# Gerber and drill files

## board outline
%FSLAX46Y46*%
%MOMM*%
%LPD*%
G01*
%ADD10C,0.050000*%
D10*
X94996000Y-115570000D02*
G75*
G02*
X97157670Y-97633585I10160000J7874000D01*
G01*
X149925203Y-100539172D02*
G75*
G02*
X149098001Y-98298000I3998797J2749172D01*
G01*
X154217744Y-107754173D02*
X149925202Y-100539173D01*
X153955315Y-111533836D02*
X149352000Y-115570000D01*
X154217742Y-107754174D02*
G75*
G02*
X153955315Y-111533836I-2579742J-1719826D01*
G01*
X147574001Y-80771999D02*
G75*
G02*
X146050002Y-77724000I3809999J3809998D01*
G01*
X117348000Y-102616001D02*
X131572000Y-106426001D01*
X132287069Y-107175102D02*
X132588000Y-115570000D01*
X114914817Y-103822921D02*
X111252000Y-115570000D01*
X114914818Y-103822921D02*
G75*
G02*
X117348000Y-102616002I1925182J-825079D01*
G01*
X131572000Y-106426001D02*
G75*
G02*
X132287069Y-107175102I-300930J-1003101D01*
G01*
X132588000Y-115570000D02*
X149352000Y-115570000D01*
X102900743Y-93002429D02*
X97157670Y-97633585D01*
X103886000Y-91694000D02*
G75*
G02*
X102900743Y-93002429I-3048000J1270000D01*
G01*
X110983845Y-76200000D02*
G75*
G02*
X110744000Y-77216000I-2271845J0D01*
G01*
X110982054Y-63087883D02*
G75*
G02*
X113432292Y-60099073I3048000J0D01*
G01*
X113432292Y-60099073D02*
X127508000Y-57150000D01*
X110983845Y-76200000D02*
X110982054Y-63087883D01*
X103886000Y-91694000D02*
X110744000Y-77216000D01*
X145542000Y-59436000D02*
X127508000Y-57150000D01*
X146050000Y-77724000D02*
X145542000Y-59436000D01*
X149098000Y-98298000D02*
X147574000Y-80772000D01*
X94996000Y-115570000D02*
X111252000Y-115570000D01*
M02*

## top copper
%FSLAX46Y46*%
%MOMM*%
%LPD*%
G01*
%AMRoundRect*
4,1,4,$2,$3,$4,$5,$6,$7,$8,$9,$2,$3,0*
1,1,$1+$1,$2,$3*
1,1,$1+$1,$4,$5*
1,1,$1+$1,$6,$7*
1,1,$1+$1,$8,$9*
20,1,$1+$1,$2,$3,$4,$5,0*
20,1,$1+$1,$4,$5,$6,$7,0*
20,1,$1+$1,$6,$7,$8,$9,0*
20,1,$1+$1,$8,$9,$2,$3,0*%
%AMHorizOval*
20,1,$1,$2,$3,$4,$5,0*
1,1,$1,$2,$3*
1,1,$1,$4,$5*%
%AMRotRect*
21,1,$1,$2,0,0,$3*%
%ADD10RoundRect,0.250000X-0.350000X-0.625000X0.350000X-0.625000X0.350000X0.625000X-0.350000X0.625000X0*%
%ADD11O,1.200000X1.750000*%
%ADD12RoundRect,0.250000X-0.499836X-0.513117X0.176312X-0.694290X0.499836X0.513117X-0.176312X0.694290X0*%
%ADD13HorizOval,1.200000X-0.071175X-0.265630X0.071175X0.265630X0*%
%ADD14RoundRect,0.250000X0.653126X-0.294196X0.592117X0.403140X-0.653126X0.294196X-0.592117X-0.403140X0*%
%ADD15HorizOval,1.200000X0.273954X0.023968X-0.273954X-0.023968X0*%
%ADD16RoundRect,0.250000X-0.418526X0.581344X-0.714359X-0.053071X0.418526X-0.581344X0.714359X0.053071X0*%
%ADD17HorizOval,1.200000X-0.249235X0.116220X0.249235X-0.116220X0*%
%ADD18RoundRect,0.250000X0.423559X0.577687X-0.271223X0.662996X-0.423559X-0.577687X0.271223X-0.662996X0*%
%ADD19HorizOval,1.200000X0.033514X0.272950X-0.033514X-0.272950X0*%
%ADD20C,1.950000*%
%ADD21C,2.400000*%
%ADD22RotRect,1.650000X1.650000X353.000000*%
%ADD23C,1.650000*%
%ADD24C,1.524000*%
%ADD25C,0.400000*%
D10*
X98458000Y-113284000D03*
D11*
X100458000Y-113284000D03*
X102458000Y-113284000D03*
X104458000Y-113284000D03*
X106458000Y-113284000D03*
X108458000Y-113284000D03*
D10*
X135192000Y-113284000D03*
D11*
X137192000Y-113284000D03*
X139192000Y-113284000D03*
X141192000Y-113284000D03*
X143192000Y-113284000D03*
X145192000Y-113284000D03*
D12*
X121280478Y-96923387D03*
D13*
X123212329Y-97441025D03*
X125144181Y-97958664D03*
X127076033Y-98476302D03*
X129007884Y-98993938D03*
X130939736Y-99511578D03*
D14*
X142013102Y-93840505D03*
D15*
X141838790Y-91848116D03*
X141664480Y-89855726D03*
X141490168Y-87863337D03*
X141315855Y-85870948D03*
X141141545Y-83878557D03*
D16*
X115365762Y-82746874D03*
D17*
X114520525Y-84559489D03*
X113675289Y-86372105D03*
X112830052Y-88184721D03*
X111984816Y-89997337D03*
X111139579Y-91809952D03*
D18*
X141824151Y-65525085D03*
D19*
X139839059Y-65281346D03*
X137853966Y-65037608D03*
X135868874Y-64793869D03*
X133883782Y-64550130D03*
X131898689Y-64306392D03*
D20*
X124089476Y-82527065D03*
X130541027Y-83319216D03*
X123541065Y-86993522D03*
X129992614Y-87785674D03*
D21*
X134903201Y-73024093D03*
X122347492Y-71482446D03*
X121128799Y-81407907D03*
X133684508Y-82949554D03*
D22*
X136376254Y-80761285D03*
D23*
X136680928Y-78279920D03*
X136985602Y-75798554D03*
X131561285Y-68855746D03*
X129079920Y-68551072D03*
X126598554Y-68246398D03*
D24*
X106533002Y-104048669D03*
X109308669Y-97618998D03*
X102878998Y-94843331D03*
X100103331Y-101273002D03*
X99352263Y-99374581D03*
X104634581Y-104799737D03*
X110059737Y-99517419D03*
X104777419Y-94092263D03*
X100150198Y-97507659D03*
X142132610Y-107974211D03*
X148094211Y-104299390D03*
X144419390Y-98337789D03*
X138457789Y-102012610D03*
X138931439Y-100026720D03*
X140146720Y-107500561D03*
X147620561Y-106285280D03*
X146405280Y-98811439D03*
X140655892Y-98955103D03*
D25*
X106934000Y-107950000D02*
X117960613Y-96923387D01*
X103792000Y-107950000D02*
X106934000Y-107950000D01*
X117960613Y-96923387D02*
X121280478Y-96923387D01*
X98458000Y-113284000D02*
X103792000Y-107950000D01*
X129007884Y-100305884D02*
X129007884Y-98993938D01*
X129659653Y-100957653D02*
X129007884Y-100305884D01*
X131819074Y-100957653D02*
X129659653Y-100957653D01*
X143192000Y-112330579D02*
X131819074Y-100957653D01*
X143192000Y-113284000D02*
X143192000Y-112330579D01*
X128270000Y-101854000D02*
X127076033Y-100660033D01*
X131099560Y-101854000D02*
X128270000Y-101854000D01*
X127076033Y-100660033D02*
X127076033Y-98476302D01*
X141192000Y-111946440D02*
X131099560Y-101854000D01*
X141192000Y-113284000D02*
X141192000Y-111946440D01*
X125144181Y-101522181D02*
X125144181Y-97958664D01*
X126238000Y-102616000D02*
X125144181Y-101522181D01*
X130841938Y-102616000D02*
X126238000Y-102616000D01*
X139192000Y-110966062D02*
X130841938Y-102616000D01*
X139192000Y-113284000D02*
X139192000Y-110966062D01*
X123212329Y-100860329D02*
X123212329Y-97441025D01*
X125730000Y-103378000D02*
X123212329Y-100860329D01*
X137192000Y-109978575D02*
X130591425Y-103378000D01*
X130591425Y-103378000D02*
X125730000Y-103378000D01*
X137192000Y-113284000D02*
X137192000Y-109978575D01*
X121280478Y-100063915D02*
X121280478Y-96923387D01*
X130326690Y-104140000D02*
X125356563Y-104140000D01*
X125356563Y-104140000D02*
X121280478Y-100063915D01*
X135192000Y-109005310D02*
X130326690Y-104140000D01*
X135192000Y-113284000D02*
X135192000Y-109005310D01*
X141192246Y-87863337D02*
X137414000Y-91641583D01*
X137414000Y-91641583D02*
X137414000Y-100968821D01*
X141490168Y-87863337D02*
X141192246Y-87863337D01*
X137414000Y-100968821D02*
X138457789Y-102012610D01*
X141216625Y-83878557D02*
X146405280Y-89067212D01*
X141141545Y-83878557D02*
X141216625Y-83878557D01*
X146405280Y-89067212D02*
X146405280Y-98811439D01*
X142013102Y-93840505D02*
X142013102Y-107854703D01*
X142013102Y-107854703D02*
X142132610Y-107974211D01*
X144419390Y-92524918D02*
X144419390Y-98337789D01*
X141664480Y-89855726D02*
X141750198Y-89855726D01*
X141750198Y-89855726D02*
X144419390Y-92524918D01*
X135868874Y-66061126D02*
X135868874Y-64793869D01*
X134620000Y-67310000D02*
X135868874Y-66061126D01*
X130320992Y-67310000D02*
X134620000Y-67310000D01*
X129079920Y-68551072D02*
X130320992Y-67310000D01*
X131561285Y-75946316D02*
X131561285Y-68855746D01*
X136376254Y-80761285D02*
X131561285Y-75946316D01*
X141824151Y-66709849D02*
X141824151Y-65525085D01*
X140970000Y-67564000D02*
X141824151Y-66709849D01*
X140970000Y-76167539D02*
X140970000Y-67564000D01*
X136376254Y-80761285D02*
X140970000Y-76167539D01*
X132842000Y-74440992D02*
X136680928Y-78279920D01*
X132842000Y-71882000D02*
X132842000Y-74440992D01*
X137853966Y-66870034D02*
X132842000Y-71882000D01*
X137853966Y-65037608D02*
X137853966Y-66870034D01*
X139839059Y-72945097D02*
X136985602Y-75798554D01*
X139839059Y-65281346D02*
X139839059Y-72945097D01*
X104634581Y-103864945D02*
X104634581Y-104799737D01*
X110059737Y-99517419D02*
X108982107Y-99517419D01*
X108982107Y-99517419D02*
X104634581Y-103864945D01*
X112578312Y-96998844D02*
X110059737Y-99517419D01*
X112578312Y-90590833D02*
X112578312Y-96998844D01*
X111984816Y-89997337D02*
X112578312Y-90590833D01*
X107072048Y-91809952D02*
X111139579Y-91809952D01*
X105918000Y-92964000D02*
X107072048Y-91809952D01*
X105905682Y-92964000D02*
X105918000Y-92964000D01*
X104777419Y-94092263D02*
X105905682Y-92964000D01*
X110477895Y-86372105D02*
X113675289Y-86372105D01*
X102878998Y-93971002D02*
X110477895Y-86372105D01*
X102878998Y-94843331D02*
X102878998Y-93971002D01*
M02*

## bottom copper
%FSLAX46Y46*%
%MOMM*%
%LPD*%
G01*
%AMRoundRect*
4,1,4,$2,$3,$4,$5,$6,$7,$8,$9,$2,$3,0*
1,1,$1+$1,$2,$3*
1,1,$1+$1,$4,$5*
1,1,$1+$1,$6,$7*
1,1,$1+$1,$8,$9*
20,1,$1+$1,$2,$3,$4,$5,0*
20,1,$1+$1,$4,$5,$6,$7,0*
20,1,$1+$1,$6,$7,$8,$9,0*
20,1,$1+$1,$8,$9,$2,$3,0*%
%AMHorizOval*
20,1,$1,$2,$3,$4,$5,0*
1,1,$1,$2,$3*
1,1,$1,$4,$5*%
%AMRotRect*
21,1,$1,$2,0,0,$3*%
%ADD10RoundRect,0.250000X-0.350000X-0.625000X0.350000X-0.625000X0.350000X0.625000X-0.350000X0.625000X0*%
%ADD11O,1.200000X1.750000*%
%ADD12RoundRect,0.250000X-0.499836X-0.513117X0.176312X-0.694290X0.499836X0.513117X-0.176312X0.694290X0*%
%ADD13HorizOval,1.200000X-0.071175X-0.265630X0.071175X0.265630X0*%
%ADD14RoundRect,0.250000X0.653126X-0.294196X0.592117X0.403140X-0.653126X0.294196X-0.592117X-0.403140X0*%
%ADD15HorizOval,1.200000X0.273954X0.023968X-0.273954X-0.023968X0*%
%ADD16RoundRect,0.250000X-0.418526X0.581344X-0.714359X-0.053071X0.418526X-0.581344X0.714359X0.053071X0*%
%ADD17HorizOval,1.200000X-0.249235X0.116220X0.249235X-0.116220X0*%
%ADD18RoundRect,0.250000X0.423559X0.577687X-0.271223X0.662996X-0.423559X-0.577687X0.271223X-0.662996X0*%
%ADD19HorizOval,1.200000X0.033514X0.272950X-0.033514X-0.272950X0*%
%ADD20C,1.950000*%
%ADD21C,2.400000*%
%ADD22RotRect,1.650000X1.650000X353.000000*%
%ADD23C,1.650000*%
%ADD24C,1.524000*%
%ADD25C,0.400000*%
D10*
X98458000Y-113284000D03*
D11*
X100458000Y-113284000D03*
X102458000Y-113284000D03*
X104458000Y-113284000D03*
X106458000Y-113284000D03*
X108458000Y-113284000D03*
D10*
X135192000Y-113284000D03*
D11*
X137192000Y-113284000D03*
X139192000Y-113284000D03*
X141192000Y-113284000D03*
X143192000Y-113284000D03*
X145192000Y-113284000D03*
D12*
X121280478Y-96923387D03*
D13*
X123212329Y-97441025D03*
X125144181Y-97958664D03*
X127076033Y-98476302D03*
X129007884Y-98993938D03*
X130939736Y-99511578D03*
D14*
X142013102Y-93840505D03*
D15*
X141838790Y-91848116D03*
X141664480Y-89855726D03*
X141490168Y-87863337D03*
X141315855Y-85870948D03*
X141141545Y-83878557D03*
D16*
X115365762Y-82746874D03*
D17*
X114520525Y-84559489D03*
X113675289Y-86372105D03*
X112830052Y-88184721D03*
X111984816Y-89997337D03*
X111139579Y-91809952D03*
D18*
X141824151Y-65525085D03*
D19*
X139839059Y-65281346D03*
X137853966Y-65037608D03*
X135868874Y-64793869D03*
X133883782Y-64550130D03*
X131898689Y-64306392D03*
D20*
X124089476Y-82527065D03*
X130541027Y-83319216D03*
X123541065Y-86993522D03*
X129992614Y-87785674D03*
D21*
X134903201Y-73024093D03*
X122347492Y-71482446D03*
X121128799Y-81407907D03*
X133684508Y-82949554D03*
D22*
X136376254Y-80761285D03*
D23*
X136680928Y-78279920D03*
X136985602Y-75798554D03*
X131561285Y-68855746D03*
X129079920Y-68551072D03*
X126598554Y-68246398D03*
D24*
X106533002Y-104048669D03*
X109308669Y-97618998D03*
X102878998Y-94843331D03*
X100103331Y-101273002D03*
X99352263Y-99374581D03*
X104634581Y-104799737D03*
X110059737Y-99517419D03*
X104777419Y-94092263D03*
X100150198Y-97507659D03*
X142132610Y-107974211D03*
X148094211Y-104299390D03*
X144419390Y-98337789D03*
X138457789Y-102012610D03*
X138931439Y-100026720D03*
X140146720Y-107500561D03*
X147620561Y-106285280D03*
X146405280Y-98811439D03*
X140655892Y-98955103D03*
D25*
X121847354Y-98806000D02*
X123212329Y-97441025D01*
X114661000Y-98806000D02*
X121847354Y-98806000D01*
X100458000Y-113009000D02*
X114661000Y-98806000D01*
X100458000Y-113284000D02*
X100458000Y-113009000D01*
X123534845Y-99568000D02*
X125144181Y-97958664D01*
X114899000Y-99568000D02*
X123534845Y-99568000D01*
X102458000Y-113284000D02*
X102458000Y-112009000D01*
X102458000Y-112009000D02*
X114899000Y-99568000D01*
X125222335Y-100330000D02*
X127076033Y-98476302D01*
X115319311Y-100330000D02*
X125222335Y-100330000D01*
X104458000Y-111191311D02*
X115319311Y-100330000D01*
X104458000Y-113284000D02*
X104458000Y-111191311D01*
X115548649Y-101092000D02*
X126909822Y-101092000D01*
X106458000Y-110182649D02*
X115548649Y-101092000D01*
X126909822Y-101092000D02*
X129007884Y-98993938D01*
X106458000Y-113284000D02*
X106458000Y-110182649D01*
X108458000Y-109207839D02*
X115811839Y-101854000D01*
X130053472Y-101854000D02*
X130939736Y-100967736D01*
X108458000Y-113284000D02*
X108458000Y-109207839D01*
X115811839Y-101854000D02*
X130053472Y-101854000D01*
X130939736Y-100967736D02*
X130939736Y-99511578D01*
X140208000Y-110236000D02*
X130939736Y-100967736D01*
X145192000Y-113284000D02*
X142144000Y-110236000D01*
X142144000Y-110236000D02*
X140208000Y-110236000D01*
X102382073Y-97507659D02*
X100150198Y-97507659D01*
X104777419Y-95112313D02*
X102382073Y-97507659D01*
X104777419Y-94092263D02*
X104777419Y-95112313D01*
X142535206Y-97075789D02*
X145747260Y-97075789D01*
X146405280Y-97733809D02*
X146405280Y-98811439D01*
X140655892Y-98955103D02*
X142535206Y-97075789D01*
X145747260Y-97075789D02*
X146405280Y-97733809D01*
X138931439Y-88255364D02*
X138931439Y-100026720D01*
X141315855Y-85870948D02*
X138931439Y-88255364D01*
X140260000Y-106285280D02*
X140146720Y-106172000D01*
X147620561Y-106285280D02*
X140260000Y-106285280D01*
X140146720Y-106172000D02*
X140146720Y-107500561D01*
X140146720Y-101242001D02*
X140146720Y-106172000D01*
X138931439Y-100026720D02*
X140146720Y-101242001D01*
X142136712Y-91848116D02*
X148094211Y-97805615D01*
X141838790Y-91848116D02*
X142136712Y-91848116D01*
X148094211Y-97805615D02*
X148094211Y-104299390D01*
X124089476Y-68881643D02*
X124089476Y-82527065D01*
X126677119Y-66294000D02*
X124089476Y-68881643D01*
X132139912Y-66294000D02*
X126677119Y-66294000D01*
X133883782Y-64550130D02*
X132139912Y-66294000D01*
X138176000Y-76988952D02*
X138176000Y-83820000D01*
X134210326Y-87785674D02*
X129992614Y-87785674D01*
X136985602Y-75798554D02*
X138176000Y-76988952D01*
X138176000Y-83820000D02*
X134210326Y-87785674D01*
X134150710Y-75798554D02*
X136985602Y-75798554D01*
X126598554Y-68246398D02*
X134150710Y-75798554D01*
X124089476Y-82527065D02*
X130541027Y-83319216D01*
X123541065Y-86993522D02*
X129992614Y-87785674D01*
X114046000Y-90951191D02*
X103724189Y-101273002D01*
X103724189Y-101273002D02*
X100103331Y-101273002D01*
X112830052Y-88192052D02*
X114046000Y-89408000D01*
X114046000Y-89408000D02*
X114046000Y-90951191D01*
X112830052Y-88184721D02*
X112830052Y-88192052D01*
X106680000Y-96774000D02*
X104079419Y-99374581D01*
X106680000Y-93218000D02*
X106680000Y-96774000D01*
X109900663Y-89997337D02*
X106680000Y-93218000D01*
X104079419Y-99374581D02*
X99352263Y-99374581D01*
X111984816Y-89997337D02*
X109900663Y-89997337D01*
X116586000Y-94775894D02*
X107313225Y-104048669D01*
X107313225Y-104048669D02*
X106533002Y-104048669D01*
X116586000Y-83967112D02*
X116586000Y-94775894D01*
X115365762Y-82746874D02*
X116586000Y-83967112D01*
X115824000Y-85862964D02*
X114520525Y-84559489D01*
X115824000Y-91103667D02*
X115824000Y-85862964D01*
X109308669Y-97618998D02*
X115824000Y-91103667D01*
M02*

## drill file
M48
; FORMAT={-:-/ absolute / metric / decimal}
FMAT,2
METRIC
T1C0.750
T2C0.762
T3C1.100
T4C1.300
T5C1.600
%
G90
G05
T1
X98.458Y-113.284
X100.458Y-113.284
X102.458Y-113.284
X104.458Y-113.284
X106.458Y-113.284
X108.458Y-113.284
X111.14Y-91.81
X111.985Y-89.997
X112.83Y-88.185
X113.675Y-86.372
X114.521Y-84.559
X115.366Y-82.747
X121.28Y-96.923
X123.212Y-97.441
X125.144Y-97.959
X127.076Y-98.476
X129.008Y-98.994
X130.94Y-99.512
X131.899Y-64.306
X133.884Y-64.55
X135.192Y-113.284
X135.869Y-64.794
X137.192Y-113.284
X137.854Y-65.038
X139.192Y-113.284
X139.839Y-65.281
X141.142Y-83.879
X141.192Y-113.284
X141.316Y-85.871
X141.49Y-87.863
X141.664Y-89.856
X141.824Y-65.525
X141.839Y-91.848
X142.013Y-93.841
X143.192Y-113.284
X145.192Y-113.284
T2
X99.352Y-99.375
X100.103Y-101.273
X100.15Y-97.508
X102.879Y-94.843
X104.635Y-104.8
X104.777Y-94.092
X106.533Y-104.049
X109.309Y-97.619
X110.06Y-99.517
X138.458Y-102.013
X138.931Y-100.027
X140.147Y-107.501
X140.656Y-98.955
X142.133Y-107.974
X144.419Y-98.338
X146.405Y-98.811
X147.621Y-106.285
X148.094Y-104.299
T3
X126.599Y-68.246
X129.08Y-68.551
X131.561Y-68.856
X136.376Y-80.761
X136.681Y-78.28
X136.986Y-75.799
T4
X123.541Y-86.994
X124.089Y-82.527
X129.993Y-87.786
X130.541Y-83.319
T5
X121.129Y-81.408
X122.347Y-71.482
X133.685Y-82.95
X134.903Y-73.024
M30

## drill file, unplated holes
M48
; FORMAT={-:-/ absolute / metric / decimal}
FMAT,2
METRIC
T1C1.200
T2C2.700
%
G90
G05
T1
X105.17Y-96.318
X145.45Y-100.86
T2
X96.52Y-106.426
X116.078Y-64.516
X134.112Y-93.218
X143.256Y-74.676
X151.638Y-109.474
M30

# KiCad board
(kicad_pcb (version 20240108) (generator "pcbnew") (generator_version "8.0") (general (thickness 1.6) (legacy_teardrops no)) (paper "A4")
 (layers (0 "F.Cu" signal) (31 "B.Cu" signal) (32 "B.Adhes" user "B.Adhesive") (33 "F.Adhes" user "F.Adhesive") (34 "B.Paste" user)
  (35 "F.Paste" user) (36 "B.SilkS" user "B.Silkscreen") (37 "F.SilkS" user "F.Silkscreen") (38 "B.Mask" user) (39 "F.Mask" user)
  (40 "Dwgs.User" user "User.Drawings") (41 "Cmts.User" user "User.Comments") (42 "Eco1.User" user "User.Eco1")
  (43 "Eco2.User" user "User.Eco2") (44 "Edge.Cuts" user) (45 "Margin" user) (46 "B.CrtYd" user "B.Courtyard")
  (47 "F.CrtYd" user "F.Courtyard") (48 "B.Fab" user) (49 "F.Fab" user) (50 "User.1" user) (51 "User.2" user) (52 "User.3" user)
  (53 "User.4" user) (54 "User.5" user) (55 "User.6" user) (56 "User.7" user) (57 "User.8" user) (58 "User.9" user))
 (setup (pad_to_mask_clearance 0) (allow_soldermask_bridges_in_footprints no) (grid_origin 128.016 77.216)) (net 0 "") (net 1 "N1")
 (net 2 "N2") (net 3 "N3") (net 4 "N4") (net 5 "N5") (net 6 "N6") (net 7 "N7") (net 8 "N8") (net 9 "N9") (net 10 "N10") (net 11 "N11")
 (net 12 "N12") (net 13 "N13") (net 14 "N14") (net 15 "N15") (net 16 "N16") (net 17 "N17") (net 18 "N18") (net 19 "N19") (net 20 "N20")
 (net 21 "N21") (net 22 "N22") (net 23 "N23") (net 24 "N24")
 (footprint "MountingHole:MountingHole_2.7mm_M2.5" (layer "F.Cu") (at 151.638 109.474)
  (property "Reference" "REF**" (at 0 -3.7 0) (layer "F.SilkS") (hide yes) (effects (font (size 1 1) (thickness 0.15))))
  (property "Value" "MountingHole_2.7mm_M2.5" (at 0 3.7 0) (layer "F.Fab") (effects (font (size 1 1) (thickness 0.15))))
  (pad "" np_thru_hole circle (at 0 0) (size 2.7 2.7) (drill 2.7) (layers "*.Cu" "*.Mask")))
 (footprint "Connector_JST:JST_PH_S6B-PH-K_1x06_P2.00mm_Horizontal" (layer "F.Cu") (at 121.280478 96.923387 -15)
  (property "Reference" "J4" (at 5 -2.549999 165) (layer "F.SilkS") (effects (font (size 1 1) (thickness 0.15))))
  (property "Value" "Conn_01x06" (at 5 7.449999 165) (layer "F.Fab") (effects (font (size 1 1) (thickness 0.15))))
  (pad "1" thru_hole roundrect (at 0 0 345) (size 1.2 1.75) (drill 0.75) (layers "*.Cu" "*.Mask") (remove_unused_layers no)
   (roundrect_rratio 0.208333) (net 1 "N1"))
  (pad "2" thru_hole oval (at 1.999999 0 345) (size 1.2 1.75) (drill 0.75) (layers "*.Cu" "*.Mask") (remove_unused_layers no) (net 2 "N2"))
  (pad "3" thru_hole oval (at 4 0.000001 345) (size 1.2 1.75) (drill 0.75) (layers "*.Cu" "*.Mask") (remove_unused_layers no) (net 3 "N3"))
  (pad "4" thru_hole oval (at 6 0.000001 345) (size 1.2 1.75) (drill 0.75) (layers "*.Cu" "*.Mask") (remove_unused_layers no) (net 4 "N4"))
  (pad "5" thru_hole oval (at 7.999999 -0.000001 345) (size 1.2 1.75) (drill 0.75) (layers "*.Cu" "*.Mask") (remove_unused_layers no)
   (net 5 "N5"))
  (pad "6" thru_hole oval (at 10 0.000001 345) (size 1.2 1.75) (drill 0.75) (layers "*.Cu" "*.Mask") (remove_unused_layers no) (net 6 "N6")))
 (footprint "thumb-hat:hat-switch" (layer "F.Cu") (at 104.706 99.446 10)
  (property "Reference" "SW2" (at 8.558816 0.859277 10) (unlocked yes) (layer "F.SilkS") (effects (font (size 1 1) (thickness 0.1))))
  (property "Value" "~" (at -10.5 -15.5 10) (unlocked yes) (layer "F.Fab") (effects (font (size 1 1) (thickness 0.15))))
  (pad "" np_thru_hole circle (at 1.000001 -2.999999 10) (size 1.2 1.2) (drill 1.2) (layers "*.Mask"))
  (pad "1" thru_hole circle (at 1.000001 4.85 10) (size 1.524 1.524) (drill 0.762) (layers "*.Cu" "*.Mask") (remove_unused_layers no)
   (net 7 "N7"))
  (pad "2" thru_hole circle (at 4.85 -1.000001 10) (size 1.524 1.524) (drill 0.762) (layers "*.Cu" "*.Mask") (remove_unused_layers no)
   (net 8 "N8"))
  (pad "3" thru_hole circle (at -1.000001 -4.85 10) (size 1.524 1.524) (drill 0.762) (layers "*.Cu" "*.Mask") (remove_unused_layers no)
   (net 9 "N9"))
  (pad "4" thru_hole circle (at -4.85 1.000001 10) (size 1.524 1.524) (drill 0.762) (layers "*.Cu" "*.Mask") (remove_unused_layers no)
   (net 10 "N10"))
  (pad "5" thru_hole circle (at -5.26 -1.000001 10) (size 1.524 1.524) (drill 0.762) (layers "*.Cu" "*.Mask") (remove_unused_layers no)
   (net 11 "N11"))
  (pad "5" thru_hole circle (at -1.000001 5.26 10) (size 1.524 1.524) (drill 0.762) (layers "*.Cu" "*.Mask") (remove_unused_layers no)
   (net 11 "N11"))
  (pad "5" thru_hole circle (at 5.26 1.000001 10) (size 1.524 1.524) (drill 0.762) (layers "*.Cu" "*.Mask") (remove_unused_layers no)
   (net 11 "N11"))
  (pad "6" thru_hole circle (at 1.000001 -5.26 10) (size 1.524 1.524) (drill 0.762) (layers "*.Cu" "*.Mask") (remove_unused_layers no)
   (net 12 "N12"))
  (pad "7" thru_hole circle (at -4.15 -2.7 10) (size 1.524 1.524) (drill 0.762) (layers "*.Cu" "*.Mask") (remove_unused_layers no)
   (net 12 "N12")))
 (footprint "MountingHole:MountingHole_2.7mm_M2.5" (layer "F.Cu") (at 116.078 64.516)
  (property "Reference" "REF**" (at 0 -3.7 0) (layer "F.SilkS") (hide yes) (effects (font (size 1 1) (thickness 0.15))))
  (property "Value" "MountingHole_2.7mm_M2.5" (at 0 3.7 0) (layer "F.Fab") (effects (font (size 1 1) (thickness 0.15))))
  (pad "" np_thru_hole circle (at 0 0) (size 2.7 2.7) (drill 2.7) (layers "*.Cu" "*.Mask")))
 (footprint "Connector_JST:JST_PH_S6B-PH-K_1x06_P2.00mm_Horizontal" (layer "F.Cu") (at 141.824151 65.525085 173)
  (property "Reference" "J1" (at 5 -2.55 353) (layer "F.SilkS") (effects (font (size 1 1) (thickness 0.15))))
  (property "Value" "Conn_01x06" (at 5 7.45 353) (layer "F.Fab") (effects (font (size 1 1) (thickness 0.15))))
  (pad "1" thru_hole roundrect (at 0 0 173) (size 1.2 1.75) (drill 0.75) (layers "*.Cu" "*.Mask") (remove_unused_layers no)
   (roundrect_rratio 0.208333) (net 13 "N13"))
  (pad "2" thru_hole oval (at 2 0 173) (size 1.2 1.75) (drill 0.75) (layers "*.Cu" "*.Mask") (remove_unused_layers no) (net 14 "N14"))
  (pad "3" thru_hole oval (at 4 0 173) (size 1.2 1.75) (drill 0.75) (layers "*.Cu" "*.Mask") (remove_unused_layers no) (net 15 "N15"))
  (pad "4" thru_hole oval (at 6 0 173) (size 1.2 1.75) (drill 0.75) (layers "*.Cu" "*.Mask") (remove_unused_layers no) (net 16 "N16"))
  (pad "5" thru_hole oval (at 8 0 173) (size 1.2 1.75) (drill 0.75) (layers "*.Cu" "*.Mask") (remove_unused_layers no) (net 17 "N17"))
  (pad "6" thru_hole oval (at 10 0 173) (size 1.2 1.75) (drill 0.75) (layers "*.Cu" "*.Mask") (remove_unused_layers no) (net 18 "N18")))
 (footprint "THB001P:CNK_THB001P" (layer "F.Cu") (at 128.016 77.216 -7)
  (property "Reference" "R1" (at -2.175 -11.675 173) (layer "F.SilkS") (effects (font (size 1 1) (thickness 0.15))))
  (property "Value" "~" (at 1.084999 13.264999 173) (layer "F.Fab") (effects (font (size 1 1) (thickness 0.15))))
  (pad "A" thru_hole circle (at -3.25 5.75 353) (size 1.95 1.95) (drill 1.3) (layers "*.Cu" "*.Mask") (remove_unused_layers no)
   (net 17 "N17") (solder_mask_margin 0.102))
  (pad "B" thru_hole circle (at 3.250001 5.75 353) (size 1.95 1.95) (drill 1.3) (layers "*.Cu" "*.Mask") (remove_unused_layers no)
   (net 17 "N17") (solder_mask_margin 0.102))
  (pad "C" thru_hole circle (at -3.249999 10.249999 353) (size 1.95 1.95) (drill 1.3) (layers "*.Cu" "*.Mask") (remove_unused_layers no)
   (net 14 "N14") (solder_mask_margin 0.102))
  (pad "D" thru_hole circle (at 3.25 10.250001 353) (size 1.95 1.95) (drill 1.3) (layers "*.Cu" "*.Mask") (remove_unused_layers no)
   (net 14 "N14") (solder_mask_margin 0.102))
  (pad "S1" thru_hole circle (at 6.325 -5 353) (size 2.4 2.4) (drill 1.6) (layers "*.Cu" "*.Mask") (remove_unused_layers no)
   (solder_mask_margin 0.102))
  (pad "S2" thru_hole circle (at -6.325 -5 353) (size 2.4 2.4) (drill 1.6) (layers "*.Cu" "*.Mask") (remove_unused_layers no)
   (solder_mask_margin 0.102))
  (pad "S3" thru_hole circle (at -6.325 5 353) (size 2.4 2.4) (drill 1.6) (layers "*.Cu" "*.Mask") (remove_unused_layers no)
   (solder_mask_margin 0.102))
  (pad "S4" thru_hole circle (at 6.325 5 353) (size 2.4 2.4) (drill 1.6) (layers "*.Cu" "*.Mask") (remove_unused_layers no)
   (solder_mask_margin 0.102))
  (pad "VR1_1" thru_hole rect (at 8.729999 2.5 353) (size 1.65 1.65) (drill 1.1) (layers "*.Cu" "*.Mask") (remove_unused_layers no)
   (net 13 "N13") (solder_mask_margin 0.102))
  (pad "VR1_2" thru_hole circle (at 8.73 0.000001 353) (size 1.65 1.65) (drill 1.1) (layers "*.Cu" "*.Mask") (remove_unused_layers no)
   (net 15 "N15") (solder_mask_margin 0.102))
  (pad "VR1_3" thru_hole circle (at 8.730001 -2.5 353) (size 1.65 1.65) (drill 1.1) (layers "*.Cu" "*.Mask") (remove_unused_layers no)
   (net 14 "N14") (solder_mask_margin 0.102))
  (pad "VR2_1" thru_hole circle (at 2.5 -8.729999 353) (size 1.65 1.65) (drill 1.1) (layers "*.Cu" "*.Mask") (remove_unused_layers no)
   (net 13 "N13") (solder_mask_margin 0.102))
  (pad "VR2_2" thru_hole circle (at 0.000001 -8.73 353) (size 1.65 1.65) (drill 1.1) (layers "*.Cu" "*.Mask") (remove_unused_layers no)
   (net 16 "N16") (solder_mask_margin 0.102))
  (pad "VR2_3" thru_hole circle (at -2.5 -8.730001 353) (size 1.65 1.65) (drill 1.1) (layers "*.Cu" "*.Mask") (remove_unused_layers no)
   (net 14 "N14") (solder_mask_margin 0.102)))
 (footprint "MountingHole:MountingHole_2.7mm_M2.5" (layer "F.Cu") (at 134.112 93.218)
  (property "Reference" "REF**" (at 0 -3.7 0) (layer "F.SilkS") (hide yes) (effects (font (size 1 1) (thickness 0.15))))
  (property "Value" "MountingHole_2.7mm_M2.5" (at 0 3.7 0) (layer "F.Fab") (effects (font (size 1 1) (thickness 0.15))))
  (pad "" np_thru_hole circle (at 0 0) (size 2.7 2.7) (drill 2.7) (layers "*.Cu" "*.Mask")))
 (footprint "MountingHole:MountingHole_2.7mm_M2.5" (layer "F.Cu") (at 96.52 106.426)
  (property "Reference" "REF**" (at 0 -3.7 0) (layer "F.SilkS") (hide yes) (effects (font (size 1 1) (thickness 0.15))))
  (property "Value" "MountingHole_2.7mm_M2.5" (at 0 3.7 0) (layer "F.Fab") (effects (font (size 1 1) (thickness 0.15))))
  (pad "" np_thru_hole circle (at 0 0) (size 2.7 2.7) (drill 2.7) (layers "*.Cu" "*.Mask")))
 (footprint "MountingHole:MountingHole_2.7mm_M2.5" (layer "F.Cu") (at 143.256 74.676)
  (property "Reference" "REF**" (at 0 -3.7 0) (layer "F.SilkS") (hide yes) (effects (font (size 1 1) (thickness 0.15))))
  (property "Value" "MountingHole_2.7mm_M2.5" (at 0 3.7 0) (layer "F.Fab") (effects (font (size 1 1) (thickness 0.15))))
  (pad "" np_thru_hole circle (at 0 0) (size 2.7 2.7) (drill 2.7) (layers "*.Cu" "*.Mask")))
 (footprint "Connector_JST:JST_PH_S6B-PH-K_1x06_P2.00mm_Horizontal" (layer "F.Cu") (at 115.365762 82.746874 -115)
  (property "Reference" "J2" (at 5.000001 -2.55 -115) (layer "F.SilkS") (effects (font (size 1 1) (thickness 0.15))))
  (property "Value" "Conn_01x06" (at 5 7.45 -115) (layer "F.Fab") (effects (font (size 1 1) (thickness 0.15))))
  (pad "1" thru_hole roundrect (at 0 0 245) (size 1.2 1.75) (drill 0.75) (layers "*.Cu" "*.Mask") (remove_unused_layers no)
   (roundrect_rratio 0.208333) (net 7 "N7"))
  (pad "2" thru_hole oval (at 2 0.000001 245) (size 1.2 1.75) (drill 0.75) (layers "*.Cu" "*.Mask") (remove_unused_layers no) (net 8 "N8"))
  (pad "3" thru_hole oval (at 4 0 245) (size 1.2 1.75) (drill 0.75) (layers "*.Cu" "*.Mask") (remove_unused_layers no) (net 9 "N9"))
  (pad "4" thru_hole oval (at 6 0 245) (size 1.2 1.75) (drill 0.75) (layers "*.Cu" "*.Mask") (remove_unused_layers no) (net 10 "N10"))
  (pad "5" thru_hole oval (at 8.000001 0 245) (size 1.2 1.75) (drill 0.75) (layers "*.Cu" "*.Mask") (remove_unused_layers no) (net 11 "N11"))
  (pad "6" thru_hole oval (at 10 0 245) (size 1.2 1.75) (drill 0.75) (layers "*.Cu" "*.Mask") (remove_unused_layers no) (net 12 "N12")))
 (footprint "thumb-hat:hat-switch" (layer "F.Cu") (at 143.276 103.156 -25)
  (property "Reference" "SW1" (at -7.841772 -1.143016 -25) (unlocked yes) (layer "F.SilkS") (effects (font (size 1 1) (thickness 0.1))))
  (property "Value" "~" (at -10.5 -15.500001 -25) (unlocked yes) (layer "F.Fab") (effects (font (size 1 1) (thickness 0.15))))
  (pad "" np_thru_hole circle (at 1 -3 335) (size 1.2 1.2) (drill 1.2) (layers "*.Mask"))
  (pad "1" thru_hole circle (at 1.000001 4.85 335) (size 1.524 1.524) (drill 0.762) (layers "*.Cu" "*.Mask") (remove_unused_layers no)
   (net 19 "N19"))
  (pad "2" thru_hole circle (at 4.85 -1.000001 335) (size 1.524 1.524) (drill 0.762) (layers "*.Cu" "*.Mask") (remove_unused_layers no)
   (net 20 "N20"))
  (pad "3" thru_hole circle (at -1.000001 -4.85 335) (size 1.524 1.524) (drill 0.762) (layers "*.Cu" "*.Mask") (remove_unused_layers no)
   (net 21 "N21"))
  (pad "4" thru_hole circle (at -4.85 1.000001 335) (size 1.524 1.524) (drill 0.762) (layers "*.Cu" "*.Mask") (remove_unused_layers no)
   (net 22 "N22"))
  (pad "5" thru_hole circle (at -5.26 -1 335) (size 1.524 1.524) (drill 0.762) (layers "*.Cu" "*.Mask") (remove_unused_layers no)
   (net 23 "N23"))
  (pad "5" thru_hole circle (at -1 5.26 335) (size 1.524 1.524) (drill 0.762) (layers "*.Cu" "*.Mask") (remove_unused_layers no)
   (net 23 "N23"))
  (pad "5" thru_hole circle (at 5.26 1 335) (size 1.524 1.524) (drill 0.762) (layers "*.Cu" "*.Mask") (remove_unused_layers no)
   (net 23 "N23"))
  (pad "6" thru_hole circle (at 1 -5.26 335) (size 1.524 1.524) (drill 0.762) (layers "*.Cu" "*.Mask") (remove_unused_layers no)
   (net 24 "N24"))
  (pad "7" thru_hole circle (at -4.15 -2.7 335) (size 1.524 1.524) (drill 0.762) (layers "*.Cu" "*.Mask") (remove_unused_layers no)
   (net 24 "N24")))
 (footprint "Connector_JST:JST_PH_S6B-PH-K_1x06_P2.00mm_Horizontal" (layer "F.Cu") (at 142.013102 93.840505 95)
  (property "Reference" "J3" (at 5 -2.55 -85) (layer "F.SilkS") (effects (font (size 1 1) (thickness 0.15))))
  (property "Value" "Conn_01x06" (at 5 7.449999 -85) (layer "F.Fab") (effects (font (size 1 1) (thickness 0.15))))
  (pad "1" thru_hole roundrect (at 0 0 95) (size 1.2 1.75) (drill 0.75) (layers "*.Cu" "*.Mask") (remove_unused_layers no)
   (roundrect_rratio 0.208333) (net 19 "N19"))
  (pad "2" thru_hole oval (at 2 -0.000001 95) (size 1.2 1.75) (drill 0.75) (layers "*.Cu" "*.Mask") (remove_unused_layers no) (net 20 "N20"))
  (pad "3" thru_hole oval (at 4 0.000001 95) (size 1.2 1.75) (drill 0.75) (layers "*.Cu" "*.Mask") (remove_unused_layers no) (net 21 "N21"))
  (pad "4" thru_hole oval (at 6 0 95) (size 1.2 1.75) (drill 0.75) (layers "*.Cu" "*.Mask") (remove_unused_layers no) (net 22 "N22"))
  (pad "5" thru_hole oval (at 8 -0.000001 95) (size 1.2 1.75) (drill 0.75) (layers "*.Cu" "*.Mask") (remove_unused_layers no) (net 23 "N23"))
  (pad "6" thru_hole oval (at 10.000001 0.000001 95) (size 1.2 1.75) (drill 0.75) (layers "*.Cu" "*.Mask") (remove_unused_layers no)
   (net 24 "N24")))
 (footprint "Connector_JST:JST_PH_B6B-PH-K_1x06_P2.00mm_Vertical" (layer "B.Cu") (at 98.458 113.284)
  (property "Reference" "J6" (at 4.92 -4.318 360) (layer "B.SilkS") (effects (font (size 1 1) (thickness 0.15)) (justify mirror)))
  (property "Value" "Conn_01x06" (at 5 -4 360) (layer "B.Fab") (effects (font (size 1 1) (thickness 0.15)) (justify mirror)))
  (pad "1" thru_hole roundrect (at 0 0) (size 1.2 1.75) (drill 0.75) (layers "*.Cu" "*.Mask") (remove_unused_layers no)
   (roundrect_rratio 0.208333) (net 1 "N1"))
  (pad "2" thru_hole oval (at 2 0) (size 1.2 1.75) (drill 0.75) (layers "*.Cu" "*.Mask") (remove_unused_layers no) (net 2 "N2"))
  (pad "3" thru_hole oval (at 4 0) (size 1.2 1.75) (drill 0.75) (layers "*.Cu" "*.Mask") (remove_unused_layers no) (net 3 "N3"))
  (pad "4" thru_hole oval (at 6 0) (size 1.2 1.75) (drill 0.75) (layers "*.Cu" "*.Mask") (remove_unused_layers no) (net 4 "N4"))
  (pad "5" thru_hole oval (at 8 0) (size 1.2 1.75) (drill 0.75) (layers "*.Cu" "*.Mask") (remove_unused_layers no) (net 5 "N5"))
  (pad "6" thru_hole oval (at 10 0) (size 1.2 1.75) (drill 0.75) (layers "*.Cu" "*.Mask") (remove_unused_layers no) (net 6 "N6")))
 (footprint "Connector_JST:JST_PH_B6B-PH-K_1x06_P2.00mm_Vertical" (layer "B.Cu") (at 135.192 113.284)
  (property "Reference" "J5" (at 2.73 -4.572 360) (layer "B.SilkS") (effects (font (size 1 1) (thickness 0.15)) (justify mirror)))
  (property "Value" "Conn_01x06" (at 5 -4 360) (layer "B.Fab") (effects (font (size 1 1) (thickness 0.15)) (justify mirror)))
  (pad "1" thru_hole roundrect (at 0 0) (size 1.2 1.75) (drill 0.75) (layers "*.Cu" "*.Mask") (remove_unused_layers no)
   (roundrect_rratio 0.208333) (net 1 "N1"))
  (pad "2" thru_hole oval (at 2 0) (size 1.2 1.75) (drill 0.75) (layers "*.Cu" "*.Mask") (remove_unused_layers no) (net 2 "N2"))
  (pad "3" thru_hole oval (at 4 0) (size 1.2 1.75) (drill 0.75) (layers "*.Cu" "*.Mask") (remove_unused_layers no) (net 3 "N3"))
  (pad "4" thru_hole oval (at 6 0) (size 1.2 1.75) (drill 0.75) (layers "*.Cu" "*.Mask") (remove_unused_layers no) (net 4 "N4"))
  (pad "5" thru_hole oval (at 8 0) (size 1.2 1.75) (drill 0.75) (layers "*.Cu" "*.Mask") (remove_unused_layers no) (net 5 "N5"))
  (pad "6" thru_hole oval (at 10 0) (size 1.2 1.75) (drill 0.75) (layers "*.Cu" "*.Mask") (remove_unused_layers no) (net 6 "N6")))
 (gr_arc (start 110.983845 76.2) (mid 110.923071 76.721963) (end 110.744 77.216) (stroke (width 0.05) (type default)) (layer "Edge.Cuts"))
 (gr_line (start 117.348 102.616001) (end 131.572 106.426001) (stroke (width 0.05) (type default)) (layer "Edge.Cuts"))
 (gr_arc (start 114.914817 103.822921) (mid 115.909266 102.771615) (end 117.348 102.616001) (stroke (width 0.05) (type default))
  (layer "Edge.Cuts"))
 (gr_line (start 146.05 77.724) (end 145.542 59.436) (stroke (width 0.05) (type default)) (layer "Edge.Cuts"))
 (gr_line (start 154.217744 107.754173) (end 149.925202 100.539173) (stroke (width 0.05) (type default)) (layer "Edge.Cuts"))
 (gr_arc (start 94.996 115.57) (mid 92.394339 106.157984) (end 97.15767 97.633585) (stroke (width 0.05) (type default)) (layer "Edge.Cuts"))
 (gr_line (start 102.900743 93.002429) (end 97.15767 97.633585) (stroke (width 0.05) (type default)) (layer "Edge.Cuts"))
 (gr_line (start 145.542 59.436) (end 127.508 57.15) (stroke (width 0.05) (type default)) (layer "Edge.Cuts"))
 (gr_arc (start 110.982054 63.087883) (mid 111.672907 61.155485) (end 113.432292 60.099073) (stroke (width 0.05) (type default))
  (layer "Edge.Cuts"))
 (gr_line (start 153.955315 111.533836) (end 149.352 115.57) (stroke (width 0.05) (type default)) (layer "Edge.Cuts"))
 (gr_arc (start 147.574 80.772) (mid 146.564689 79.371656) (end 146.050001 77.724) (stroke (width 0.05) (type default)) (layer "Edge.Cuts"))
 (gr_line (start 149.098 98.298) (end 147.574 80.772) (stroke (width 0.05) (type default)) (layer "Edge.Cuts"))
 (gr_line (start 132.588 115.57) (end 149.352 115.57) (stroke (width 0.05) (type default)) (layer "Edge.Cuts"))
 (gr_line (start 114.914817 103.822921) (end 111.252 115.57) (stroke (width 0.05) (type default)) (layer "Edge.Cuts"))
 (gr_line (start 94.996 115.57) (end 111.252 115.57) (stroke (width 0.05) (type default)) (layer "Edge.Cuts"))
 (gr_line (start 113.432292 60.099073) (end 127.508 57.15) (stroke (width 0.05) (type default)) (layer "Edge.Cuts"))
 (gr_arc (start 103.886 91.694) (mid 103.475787 92.410274) (end 102.900743 93.002429) (stroke (width 0.05) (type default))
  (layer "Edge.Cuts"))
 (gr_line (start 132.287069 107.175102) (end 132.588 115.57) (stroke (width 0.05) (type default)) (layer "Edge.Cuts"))
 (gr_line (start 103.886 91.694) (end 110.744 77.216) (stroke (width 0.05) (type default)) (layer "Edge.Cuts"))
 (gr_arc (start 154.217743 107.754174) (mid 154.731017 109.688753) (end 153.955315 111.533836) (stroke (width 0.05) (type default))
  (layer "Edge.Cuts"))
 (gr_arc (start 131.572 106.426001) (mid 132.028608 106.705979) (end 132.287069 107.175102) (stroke (width 0.05) (type default))
  (layer "Edge.Cuts"))
 (gr_line (start 110.983845 76.2) (end 110.982054 63.087883) (stroke (width 0.05) (type default)) (layer "Edge.Cuts"))
 (gr_arc (start 149.925202 100.539173) (mid 149.371531 99.470286) (end 149.098 98.298) (stroke (width 0.05) (type default))
  (layer "Edge.Cuts"))
 (segment (start 126.677119 66.294) (end 124.089476 68.881643) (width 0.4) (layer "B.Cu") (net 17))
 (segment (start 124.089476 82.527065) (end 130.541027 83.319216) (width 0.4) (layer "B.Cu") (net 17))
 (segment (start 133.883782 64.55013) (end 132.139912 66.294) (width 0.4) (layer "B.Cu") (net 17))
 (segment (start 132.139912 66.294) (end 126.677119 66.294) (width 0.4) (layer "B.Cu") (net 17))
 (segment (start 124.089476 68.881643) (end 124.089476 82.527065) (width 0.4) (layer "B.Cu") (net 17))
 (segment (start 136.376254 80.761285) (end 140.97 76.167539) (width 0.4) (layer "F.Cu") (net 13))
 (segment (start 141.824151 66.709849) (end 141.824151 65.525085) (width 0.4) (layer "F.Cu") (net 13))
 (segment (start 140.97 76.167539) (end 140.97 67.564) (width 0.4) (layer "F.Cu") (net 13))
 (segment (start 140.97 67.564) (end 141.824151 66.709849) (width 0.4) (layer "F.Cu") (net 13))
 (segment (start 131.561285 75.946316) (end 131.561285 68.855746) (width 0.4) (layer "F.Cu") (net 13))
 (segment (start 136.376254 80.761285) (end 131.561285 75.946316) (width 0.4) (layer "F.Cu") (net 13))
 (segment (start 132.842 71.882) (end 132.842 74.440992) (width 0.4) (layer "F.Cu") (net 15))
 (segment (start 137.853966 65.037608) (end 137.853966 66.870034) (width 0.4) (layer "F.Cu") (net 15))
 (segment (start 137.853966 66.870034) (end 132.842 71.882) (width 0.4) (layer "F.Cu") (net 15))
 (segment (start 132.842 74.440992) (end 136.680928 78.27992) (width 0.4) (layer "F.Cu") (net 15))
 (segment (start 139.839059 72.945097) (end 136.985602 75.798554) (width 0.4) (layer "F.Cu") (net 14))
 (segment (start 139.839059 65.281346) (end 139.839059 72.945097) (width 0.4) (layer "F.Cu") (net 14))
 (segment (start 134.210326 87.785674) (end 129.992614 87.785674) (width 0.4) (layer "B.Cu") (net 14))
 (segment (start 134.15071 75.798554) (end 136.985602 75.798554) (width 0.4) (layer "B.Cu") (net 14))
 (segment (start 138.176 76.988952) (end 138.176 83.82) (width 0.4) (layer "B.Cu") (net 14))
 (segment (start 126.598554 68.246398) (end 134.15071 75.798554) (width 0.4) (layer "B.Cu") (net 14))
 (segment (start 123.541065 86.993522) (end 129.992614 87.785674) (width 0.4) (layer "B.Cu") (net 14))
 (segment (start 138.176 83.82) (end 134.210326 87.785674) (width 0.4) (layer "B.Cu") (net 14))
 (segment (start 136.985602 75.798554) (end 138.176 76.988952) (width 0.4) (layer "B.Cu") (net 14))
 (segment (start 130.320992 67.31) (end 134.62 67.31) (width 0.4) (layer "F.Cu") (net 16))
 (segment (start 129.07992 68.551072) (end 130.320992 67.31) (width 0.4) (layer "F.Cu") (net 16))
 (segment (start 134.62 67.31) (end 135.868874 66.061126) (width 0.4) (layer "F.Cu") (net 16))
 (segment (start 135.868874 66.061126) (end 135.868874 64.793869) (width 0.4) (layer "F.Cu") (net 16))
 (segment (start 116.586 94.775894) (end 107.313225 104.048669) (width 0.4) (layer "B.Cu") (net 7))
 (segment (start 115.365762 82.746874) (end 116.586 83.967112) (width 0.4) (layer "B.Cu") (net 7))
 (segment (start 116.586 83.967112) (end 116.586 94.775894) (width 0.4) (layer "B.Cu") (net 7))
 (segment (start 107.313225 104.048669) (end 106.533002 104.048669) (width 0.4) (layer "B.Cu") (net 7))
 (segment (start 114.046 89.408) (end 114.046 90.951191) (width 0.4) (layer "B.Cu") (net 10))
 (segment (start 112.830052 88.184721) (end 112.830052 88.192052) (width 0.4) (layer "B.Cu") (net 10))
 (segment (start 114.046 90.951191) (end 103.724189 101.273002) (width 0.4) (layer "B.Cu") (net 10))
 (segment (start 103.724189 101.273002) (end 100.103331 101.273002) (width 0.4) (layer "B.Cu") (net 10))
 (segment (start 112.830052 88.192052) (end 114.046 89.408) (width 0.4) (layer "B.Cu") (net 10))
 (segment (start 111.984816 89.997337) (end 112.578312 90.590833) (width 0.4) (layer "F.Cu") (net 11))
 (segment (start 110.059737 99.517419) (end 108.982107 99.517419) (width 0.4) (layer "F.Cu") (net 11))
 (segment (start 104.634581 103.864945) (end 104.634581 104.799737) (width 0.4) (layer "F.Cu") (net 11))
 (segment (start 112.578312 90.590833) (end 112.578312 96.998844) (width 0.4) (layer "F.Cu") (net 11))
 (segment (start 108.982107 99.517419) (end 104.634581 103.864945) (width 0.4) (layer "F.Cu") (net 11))
 (segment (start 112.578312 96.998844) (end 110.059737 99.517419) (width 0.4) (layer "F.Cu") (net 11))
 (segment (start 109.900663 89.997337) (end 106.68 93.218) (width 0.4) (layer "B.Cu") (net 11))
 (segment (start 106.68 93.218) (end 106.68 96.774) (width 0.4) (layer "B.Cu") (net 11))
 (segment (start 104.079419 99.374581) (end 99.352263 99.374581) (width 0.4) (layer "B.Cu") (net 11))
 (segment (start 106.68 96.774) (end 104.079419 99.374581) (width 0.4) (layer "B.Cu") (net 11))
 (segment (start 111.984816 89.997337) (end 109.900663 89.997337) (width 0.4) (layer "B.Cu") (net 11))
 (segment (start 104.777419 94.092263) (end 105.905682 92.964) (width 0.4) (layer "F.Cu") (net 12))
 (segment (start 107.072048 91.809952) (end 111.139579 91.809952) (width 0.4) (layer "F.Cu") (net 12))
 (segment (start 105.905682 92.964) (end 105.918 92.964) (width 0.4) (layer "F.Cu") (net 12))
 (segment (start 105.918 92.964) (end 107.072048 91.809952) (width 0.4) (layer "F.Cu") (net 12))
 (segment (start 104.777419 95.112313) (end 102.382073 97.507659) (width 0.4) (layer "B.Cu") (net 12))
 (segment (start 102.382073 97.507659) (end 100.150198 97.507659) (width 0.4) (layer "B.Cu") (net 12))
 (segment (start 104.777419 94.092263) (end 104.777419 95.112313) (width 0.4) (layer "B.Cu") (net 12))
 (segment (start 109.308669 97.618998) (end 115.824 91.103667) (width 0.4) (layer "B.Cu") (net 8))
 (segment (start 115.824 85.862964) (end 114.520525 84.559489) (width 0.4) (layer "B.Cu") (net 8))
 (segment (start 115.824 91.103667) (end 115.824 85.862964) (width 0.4) (layer "B.Cu") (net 8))
 (segment (start 110.477895 86.372105) (end 113.675289 86.372105) (width 0.4) (layer "F.Cu") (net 9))
 (segment (start 102.878998 93.971002) (end 110.477895 86.372105) (width 0.4) (layer "F.Cu") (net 9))
 (segment (start 102.878998 94.843331) (end 102.878998 93.971002) (width 0.4) (layer "F.Cu") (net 9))
 (segment (start 144.41939 92.524918) (end 144.41939 98.337789) (width 0.4) (layer "F.Cu") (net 21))
 (segment (start 141.66448 89.855726) (end 141.750198 89.855726) (width 0.4) (layer "F.Cu") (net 21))
 (segment (start 141.750198 89.855726) (end 144.41939 92.524918) (width 0.4) (layer "F.Cu") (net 21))
 (segment (start 140.14672 101.242001) (end 140.14672 106.172) (width 0.4) (layer "B.Cu") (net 23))
 (segment (start 140.14672 106.172) (end 140.14672 107.500561) (width 0.4) (layer "B.Cu") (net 23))
 (segment (start 141.315855 85.870948) (end 138.931439 88.255364) (width 0.4) (layer "B.Cu") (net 23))
 (segment (start 140.26 106.28528) (end 140.14672 106.172) (width 0.4) (layer "B.Cu") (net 23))
 (segment (start 138.931439 88.255364) (end 138.931439 100.02672) (width 0.4) (layer "B.Cu") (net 23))
 (segment (start 147.620561 106.28528) (end 140.26 106.28528) (width 0.4) (layer "B.Cu") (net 23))
 (segment (start 138.931439 100.02672) (end 140.14672 101.242001) (width 0.4) (layer "B.Cu") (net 23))
 (segment (start 141.490168 87.863337) (end 141.192246 87.863337) (width 0.4) (layer "F.Cu") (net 22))
 (segment (start 137.414 100.968821) (end 138.457789 102.01261) (width 0.4) (layer "F.Cu") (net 22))
 (segment (start 141.192246 87.863337) (end 137.414 91.641583) (width 0.4) (layer "F.Cu") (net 22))
 (segment (start 137.414 91.641583) (end 137.414 100.968821) (width 0.4) (layer "F.Cu") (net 22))
 (segment (start 142.013102 93.840505) (end 142.013102 107.854703) (width 0.4) (layer "F.Cu") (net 19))
 (segment (start 142.013102 107.854703) (end 142.13261 107.974211) (width 0.4) (layer "F.Cu") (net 19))
 (segment (start 148.094211 97.805615) (end 148.094211 104.29939) (width 0.4) (layer "B.Cu") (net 20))
 (segment (start 142.136712 91.848116) (end 148.094211 97.805615) (width 0.4) (layer "B.Cu") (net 20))
 (segment (start 141.83879 91.848116) (end 142.136712 91.848116) (width 0.4) (layer "B.Cu") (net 20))
 (segment (start 141.216625 83.878557) (end 146.40528 89.067212) (width 0.4) (layer "F.Cu") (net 24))
 (segment (start 146.40528 89.067212) (end 146.40528 98.811439) (width 0.4) (layer "F.Cu") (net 24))
 (segment (start 141.141545 83.878557) (end 141.216625 83.878557) (width 0.4) (layer "F.Cu") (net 24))
 (segment (start 140.655892 98.955103) (end 142.535206 97.075789) (width 0.4) (layer "B.Cu") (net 24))
 (segment (start 145.74726 97.075789) (end 146.40528 97.733809) (width 0.4) (layer "B.Cu") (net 24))
 (segment (start 146.40528 97.733809) (end 146.40528 98.811439) (width 0.4) (layer "B.Cu") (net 24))
 (segment (start 142.535206 97.075789) (end 145.74726 97.075789) (width 0.4) (layer "B.Cu") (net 24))
 (segment (start 103.792 107.95) (end 106.934 107.95) (width 0.4) (layer "F.Cu") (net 1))
 (segment (start 125.356563 104.14) (end 121.280478 100.063915) (width 0.4) (layer "F.Cu") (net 1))
 (segment (start 98.458 113.284) (end 103.792 107.95) (width 0.4) (layer "F.Cu") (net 1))
 (segment (start 135.192 113.284) (end 135.192 109.00531) (width 0.4) (layer "F.Cu") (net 1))
 (segment (start 117.960613 96.923387) (end 121.280478 96.923387) (width 0.4) (layer "F.Cu") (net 1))
 (segment (start 121.280478 100.063915) (end 121.280478 96.923387) (width 0.4) (layer "F.Cu") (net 1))
 (segment (start 130.32669 104.14) (end 125.356563 104.14) (width 0.4) (layer "F.Cu") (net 1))
 (segment (start 106.934 107.95) (end 117.960613 96.923387) (width 0.4) (layer "F.Cu") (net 1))
 (segment (start 135.192 109.00531) (end 130.32669 104.14) (width 0.4) (layer "F.Cu") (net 1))
 (segment (start 139.192 113.284) (end 139.192 110.966062) (width 0.4) (layer "F.Cu") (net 3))
 (segment (start 126.238 102.616) (end 125.144181 101.522181) (width 0.4) (layer "F.Cu") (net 3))
 (segment (start 130.841938 102.616) (end 126.238 102.616) (width 0.4) (layer "F.Cu") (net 3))
 (segment (start 139.192 110.966062) (end 130.841938 102.616) (width 0.4) (layer "F.Cu") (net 3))
 (segment (start 125.144181 101.522181) (end 125.144181 97.958664) (width 0.4) (layer "F.Cu") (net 3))
 (segment (start 123.534845 99.568) (end 125.144181 97.958664) (width 0.4) (layer "B.Cu") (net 3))
 (segment (start 114.899 99.568) (end 123.534845 99.568) (width 0.4) (layer "B.Cu") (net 3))
 (segment (start 102.458 112.009) (end 114.899 99.568) (width 0.4) (layer "B.Cu") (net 3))
 (segment (start 102.458 113.284) (end 102.458 112.009) (width 0.4) (layer "B.Cu") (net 3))
 (segment (start 128.27 101.854) (end 127.076033 100.660033) (width 0.4) (layer "F.Cu") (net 4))
 (segment (start 127.076033 100.660033) (end 127.076033 98.476302) (width 0.4) (layer "F.Cu") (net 4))
 (segment (start 131.09956 101.854) (end 128.27 101.854) (width 0.4) (layer "F.Cu") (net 4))
 (segment (start 141.192 111.94644) (end 131.09956 101.854) (width 0.4) (layer "F.Cu") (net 4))
 (segment (start 141.192 113.284) (end 141.192 111.94644) (width 0.4) (layer "F.Cu") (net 4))
 (segment (start 115.319311 100.33) (end 125.222335 100.33) (width 0.4) (layer "B.Cu") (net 4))
 (segment (start 104.458 113.284) (end 104.458 111.191311) (width 0.4) (layer "B.Cu") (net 4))
 (segment (start 104.458 111.191311) (end 115.319311 100.33) (width 0.4) (layer "B.Cu") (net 4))
 (segment (start 125.222335 100.33) (end 127.076033 98.476302) (width 0.4) (layer "B.Cu") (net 4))
 (segment (start 143.192 112.330579) (end 131.819074 100.957653) (width 0.4) (layer "F.Cu") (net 5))
 (segment (start 143.192 113.284) (end 143.192 112.330579) (width 0.4) (layer "F.Cu") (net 5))
 (segment (start 129.007884 100.305884) (end 129.007884 98.993938) (width 0.4) (layer "F.Cu") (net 5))
 (segment (start 129.659653 100.957653) (end 129.007884 100.305884) (width 0.4) (layer "F.Cu") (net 5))
 (segment (start 131.819074 100.957653) (end 129.659653 100.957653) (width 0.4) (layer "F.Cu") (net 5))
 (segment (start 126.909822 101.092) (end 129.007884 98.993938) (width 0.4) (layer "B.Cu") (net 5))
 (segment (start 115.548649 101.092) (end 126.909822 101.092) (width 0.4) (layer "B.Cu") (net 5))
 (segment (start 106.458 113.284) (end 106.458 110.182649) (width 0.4) (layer "B.Cu") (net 5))
 (segment (start 106.458 110.182649) (end 115.548649 101.092) (width 0.4) (layer "B.Cu") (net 5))
 (segment (start 123.212329 100.860329) (end 123.212329 97.441025) (width 0.4) (layer "F.Cu") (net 2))
 (segment (start 137.192 109.978575) (end 130.591425 103.378) (width 0.4) (layer "F.Cu") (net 2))
 (segment (start 125.73 103.378) (end 123.212329 100.860329) (width 0.4) (layer "F.Cu") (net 2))
 (segment (start 130.591425 103.378) (end 125.73 103.378) (width 0.4) (layer "F.Cu") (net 2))
 (segment (start 137.192 113.284) (end 137.192 109.978575) (width 0.4) (layer "F.Cu") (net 2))
 (segment (start 100.458 113.009) (end 114.661 98.806) (width 0.4) (layer "B.Cu") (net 2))
 (segment (start 114.661 98.806) (end 121.847354 98.806) (width 0.4) (layer "B.Cu") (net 2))
 (segment (start 121.847354 98.806) (end 123.212329 97.441025) (width 0.4) (layer "B.Cu") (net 2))
 (segment (start 100.458 113.284) (end 100.458 113.009) (width 0.4) (layer "B.Cu") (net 2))
 (segment (start 130.053472 101.854) (end 130.939736 100.967736) (width 0.4) (layer "B.Cu") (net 6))
 (segment (start 108.458 113.284) (end 108.458 109.207839) (width 0.4) (layer "B.Cu") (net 6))
 (segment (start 140.208 110.236) (end 130.939736 100.967736) (width 0.4) (layer "B.Cu") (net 6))
 (segment (start 108.458 109.207839) (end 115.811839 101.854) (width 0.4) (layer "B.Cu") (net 6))
 (segment (start 115.811839 101.854) (end 130.053472 101.854) (width 0.4) (layer "B.Cu") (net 6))
 (segment (start 142.144 110.236) (end 140.208 110.236) (width 0.4) (layer "B.Cu") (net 6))
 (segment (start 145.192 113.284) (end 142.144 110.236) (width 0.4) (layer "B.Cu") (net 6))
 (segment (start 130.939736 100.967736) (end 130.939736 99.511578) (width 0.4) (layer "B.Cu") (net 6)))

